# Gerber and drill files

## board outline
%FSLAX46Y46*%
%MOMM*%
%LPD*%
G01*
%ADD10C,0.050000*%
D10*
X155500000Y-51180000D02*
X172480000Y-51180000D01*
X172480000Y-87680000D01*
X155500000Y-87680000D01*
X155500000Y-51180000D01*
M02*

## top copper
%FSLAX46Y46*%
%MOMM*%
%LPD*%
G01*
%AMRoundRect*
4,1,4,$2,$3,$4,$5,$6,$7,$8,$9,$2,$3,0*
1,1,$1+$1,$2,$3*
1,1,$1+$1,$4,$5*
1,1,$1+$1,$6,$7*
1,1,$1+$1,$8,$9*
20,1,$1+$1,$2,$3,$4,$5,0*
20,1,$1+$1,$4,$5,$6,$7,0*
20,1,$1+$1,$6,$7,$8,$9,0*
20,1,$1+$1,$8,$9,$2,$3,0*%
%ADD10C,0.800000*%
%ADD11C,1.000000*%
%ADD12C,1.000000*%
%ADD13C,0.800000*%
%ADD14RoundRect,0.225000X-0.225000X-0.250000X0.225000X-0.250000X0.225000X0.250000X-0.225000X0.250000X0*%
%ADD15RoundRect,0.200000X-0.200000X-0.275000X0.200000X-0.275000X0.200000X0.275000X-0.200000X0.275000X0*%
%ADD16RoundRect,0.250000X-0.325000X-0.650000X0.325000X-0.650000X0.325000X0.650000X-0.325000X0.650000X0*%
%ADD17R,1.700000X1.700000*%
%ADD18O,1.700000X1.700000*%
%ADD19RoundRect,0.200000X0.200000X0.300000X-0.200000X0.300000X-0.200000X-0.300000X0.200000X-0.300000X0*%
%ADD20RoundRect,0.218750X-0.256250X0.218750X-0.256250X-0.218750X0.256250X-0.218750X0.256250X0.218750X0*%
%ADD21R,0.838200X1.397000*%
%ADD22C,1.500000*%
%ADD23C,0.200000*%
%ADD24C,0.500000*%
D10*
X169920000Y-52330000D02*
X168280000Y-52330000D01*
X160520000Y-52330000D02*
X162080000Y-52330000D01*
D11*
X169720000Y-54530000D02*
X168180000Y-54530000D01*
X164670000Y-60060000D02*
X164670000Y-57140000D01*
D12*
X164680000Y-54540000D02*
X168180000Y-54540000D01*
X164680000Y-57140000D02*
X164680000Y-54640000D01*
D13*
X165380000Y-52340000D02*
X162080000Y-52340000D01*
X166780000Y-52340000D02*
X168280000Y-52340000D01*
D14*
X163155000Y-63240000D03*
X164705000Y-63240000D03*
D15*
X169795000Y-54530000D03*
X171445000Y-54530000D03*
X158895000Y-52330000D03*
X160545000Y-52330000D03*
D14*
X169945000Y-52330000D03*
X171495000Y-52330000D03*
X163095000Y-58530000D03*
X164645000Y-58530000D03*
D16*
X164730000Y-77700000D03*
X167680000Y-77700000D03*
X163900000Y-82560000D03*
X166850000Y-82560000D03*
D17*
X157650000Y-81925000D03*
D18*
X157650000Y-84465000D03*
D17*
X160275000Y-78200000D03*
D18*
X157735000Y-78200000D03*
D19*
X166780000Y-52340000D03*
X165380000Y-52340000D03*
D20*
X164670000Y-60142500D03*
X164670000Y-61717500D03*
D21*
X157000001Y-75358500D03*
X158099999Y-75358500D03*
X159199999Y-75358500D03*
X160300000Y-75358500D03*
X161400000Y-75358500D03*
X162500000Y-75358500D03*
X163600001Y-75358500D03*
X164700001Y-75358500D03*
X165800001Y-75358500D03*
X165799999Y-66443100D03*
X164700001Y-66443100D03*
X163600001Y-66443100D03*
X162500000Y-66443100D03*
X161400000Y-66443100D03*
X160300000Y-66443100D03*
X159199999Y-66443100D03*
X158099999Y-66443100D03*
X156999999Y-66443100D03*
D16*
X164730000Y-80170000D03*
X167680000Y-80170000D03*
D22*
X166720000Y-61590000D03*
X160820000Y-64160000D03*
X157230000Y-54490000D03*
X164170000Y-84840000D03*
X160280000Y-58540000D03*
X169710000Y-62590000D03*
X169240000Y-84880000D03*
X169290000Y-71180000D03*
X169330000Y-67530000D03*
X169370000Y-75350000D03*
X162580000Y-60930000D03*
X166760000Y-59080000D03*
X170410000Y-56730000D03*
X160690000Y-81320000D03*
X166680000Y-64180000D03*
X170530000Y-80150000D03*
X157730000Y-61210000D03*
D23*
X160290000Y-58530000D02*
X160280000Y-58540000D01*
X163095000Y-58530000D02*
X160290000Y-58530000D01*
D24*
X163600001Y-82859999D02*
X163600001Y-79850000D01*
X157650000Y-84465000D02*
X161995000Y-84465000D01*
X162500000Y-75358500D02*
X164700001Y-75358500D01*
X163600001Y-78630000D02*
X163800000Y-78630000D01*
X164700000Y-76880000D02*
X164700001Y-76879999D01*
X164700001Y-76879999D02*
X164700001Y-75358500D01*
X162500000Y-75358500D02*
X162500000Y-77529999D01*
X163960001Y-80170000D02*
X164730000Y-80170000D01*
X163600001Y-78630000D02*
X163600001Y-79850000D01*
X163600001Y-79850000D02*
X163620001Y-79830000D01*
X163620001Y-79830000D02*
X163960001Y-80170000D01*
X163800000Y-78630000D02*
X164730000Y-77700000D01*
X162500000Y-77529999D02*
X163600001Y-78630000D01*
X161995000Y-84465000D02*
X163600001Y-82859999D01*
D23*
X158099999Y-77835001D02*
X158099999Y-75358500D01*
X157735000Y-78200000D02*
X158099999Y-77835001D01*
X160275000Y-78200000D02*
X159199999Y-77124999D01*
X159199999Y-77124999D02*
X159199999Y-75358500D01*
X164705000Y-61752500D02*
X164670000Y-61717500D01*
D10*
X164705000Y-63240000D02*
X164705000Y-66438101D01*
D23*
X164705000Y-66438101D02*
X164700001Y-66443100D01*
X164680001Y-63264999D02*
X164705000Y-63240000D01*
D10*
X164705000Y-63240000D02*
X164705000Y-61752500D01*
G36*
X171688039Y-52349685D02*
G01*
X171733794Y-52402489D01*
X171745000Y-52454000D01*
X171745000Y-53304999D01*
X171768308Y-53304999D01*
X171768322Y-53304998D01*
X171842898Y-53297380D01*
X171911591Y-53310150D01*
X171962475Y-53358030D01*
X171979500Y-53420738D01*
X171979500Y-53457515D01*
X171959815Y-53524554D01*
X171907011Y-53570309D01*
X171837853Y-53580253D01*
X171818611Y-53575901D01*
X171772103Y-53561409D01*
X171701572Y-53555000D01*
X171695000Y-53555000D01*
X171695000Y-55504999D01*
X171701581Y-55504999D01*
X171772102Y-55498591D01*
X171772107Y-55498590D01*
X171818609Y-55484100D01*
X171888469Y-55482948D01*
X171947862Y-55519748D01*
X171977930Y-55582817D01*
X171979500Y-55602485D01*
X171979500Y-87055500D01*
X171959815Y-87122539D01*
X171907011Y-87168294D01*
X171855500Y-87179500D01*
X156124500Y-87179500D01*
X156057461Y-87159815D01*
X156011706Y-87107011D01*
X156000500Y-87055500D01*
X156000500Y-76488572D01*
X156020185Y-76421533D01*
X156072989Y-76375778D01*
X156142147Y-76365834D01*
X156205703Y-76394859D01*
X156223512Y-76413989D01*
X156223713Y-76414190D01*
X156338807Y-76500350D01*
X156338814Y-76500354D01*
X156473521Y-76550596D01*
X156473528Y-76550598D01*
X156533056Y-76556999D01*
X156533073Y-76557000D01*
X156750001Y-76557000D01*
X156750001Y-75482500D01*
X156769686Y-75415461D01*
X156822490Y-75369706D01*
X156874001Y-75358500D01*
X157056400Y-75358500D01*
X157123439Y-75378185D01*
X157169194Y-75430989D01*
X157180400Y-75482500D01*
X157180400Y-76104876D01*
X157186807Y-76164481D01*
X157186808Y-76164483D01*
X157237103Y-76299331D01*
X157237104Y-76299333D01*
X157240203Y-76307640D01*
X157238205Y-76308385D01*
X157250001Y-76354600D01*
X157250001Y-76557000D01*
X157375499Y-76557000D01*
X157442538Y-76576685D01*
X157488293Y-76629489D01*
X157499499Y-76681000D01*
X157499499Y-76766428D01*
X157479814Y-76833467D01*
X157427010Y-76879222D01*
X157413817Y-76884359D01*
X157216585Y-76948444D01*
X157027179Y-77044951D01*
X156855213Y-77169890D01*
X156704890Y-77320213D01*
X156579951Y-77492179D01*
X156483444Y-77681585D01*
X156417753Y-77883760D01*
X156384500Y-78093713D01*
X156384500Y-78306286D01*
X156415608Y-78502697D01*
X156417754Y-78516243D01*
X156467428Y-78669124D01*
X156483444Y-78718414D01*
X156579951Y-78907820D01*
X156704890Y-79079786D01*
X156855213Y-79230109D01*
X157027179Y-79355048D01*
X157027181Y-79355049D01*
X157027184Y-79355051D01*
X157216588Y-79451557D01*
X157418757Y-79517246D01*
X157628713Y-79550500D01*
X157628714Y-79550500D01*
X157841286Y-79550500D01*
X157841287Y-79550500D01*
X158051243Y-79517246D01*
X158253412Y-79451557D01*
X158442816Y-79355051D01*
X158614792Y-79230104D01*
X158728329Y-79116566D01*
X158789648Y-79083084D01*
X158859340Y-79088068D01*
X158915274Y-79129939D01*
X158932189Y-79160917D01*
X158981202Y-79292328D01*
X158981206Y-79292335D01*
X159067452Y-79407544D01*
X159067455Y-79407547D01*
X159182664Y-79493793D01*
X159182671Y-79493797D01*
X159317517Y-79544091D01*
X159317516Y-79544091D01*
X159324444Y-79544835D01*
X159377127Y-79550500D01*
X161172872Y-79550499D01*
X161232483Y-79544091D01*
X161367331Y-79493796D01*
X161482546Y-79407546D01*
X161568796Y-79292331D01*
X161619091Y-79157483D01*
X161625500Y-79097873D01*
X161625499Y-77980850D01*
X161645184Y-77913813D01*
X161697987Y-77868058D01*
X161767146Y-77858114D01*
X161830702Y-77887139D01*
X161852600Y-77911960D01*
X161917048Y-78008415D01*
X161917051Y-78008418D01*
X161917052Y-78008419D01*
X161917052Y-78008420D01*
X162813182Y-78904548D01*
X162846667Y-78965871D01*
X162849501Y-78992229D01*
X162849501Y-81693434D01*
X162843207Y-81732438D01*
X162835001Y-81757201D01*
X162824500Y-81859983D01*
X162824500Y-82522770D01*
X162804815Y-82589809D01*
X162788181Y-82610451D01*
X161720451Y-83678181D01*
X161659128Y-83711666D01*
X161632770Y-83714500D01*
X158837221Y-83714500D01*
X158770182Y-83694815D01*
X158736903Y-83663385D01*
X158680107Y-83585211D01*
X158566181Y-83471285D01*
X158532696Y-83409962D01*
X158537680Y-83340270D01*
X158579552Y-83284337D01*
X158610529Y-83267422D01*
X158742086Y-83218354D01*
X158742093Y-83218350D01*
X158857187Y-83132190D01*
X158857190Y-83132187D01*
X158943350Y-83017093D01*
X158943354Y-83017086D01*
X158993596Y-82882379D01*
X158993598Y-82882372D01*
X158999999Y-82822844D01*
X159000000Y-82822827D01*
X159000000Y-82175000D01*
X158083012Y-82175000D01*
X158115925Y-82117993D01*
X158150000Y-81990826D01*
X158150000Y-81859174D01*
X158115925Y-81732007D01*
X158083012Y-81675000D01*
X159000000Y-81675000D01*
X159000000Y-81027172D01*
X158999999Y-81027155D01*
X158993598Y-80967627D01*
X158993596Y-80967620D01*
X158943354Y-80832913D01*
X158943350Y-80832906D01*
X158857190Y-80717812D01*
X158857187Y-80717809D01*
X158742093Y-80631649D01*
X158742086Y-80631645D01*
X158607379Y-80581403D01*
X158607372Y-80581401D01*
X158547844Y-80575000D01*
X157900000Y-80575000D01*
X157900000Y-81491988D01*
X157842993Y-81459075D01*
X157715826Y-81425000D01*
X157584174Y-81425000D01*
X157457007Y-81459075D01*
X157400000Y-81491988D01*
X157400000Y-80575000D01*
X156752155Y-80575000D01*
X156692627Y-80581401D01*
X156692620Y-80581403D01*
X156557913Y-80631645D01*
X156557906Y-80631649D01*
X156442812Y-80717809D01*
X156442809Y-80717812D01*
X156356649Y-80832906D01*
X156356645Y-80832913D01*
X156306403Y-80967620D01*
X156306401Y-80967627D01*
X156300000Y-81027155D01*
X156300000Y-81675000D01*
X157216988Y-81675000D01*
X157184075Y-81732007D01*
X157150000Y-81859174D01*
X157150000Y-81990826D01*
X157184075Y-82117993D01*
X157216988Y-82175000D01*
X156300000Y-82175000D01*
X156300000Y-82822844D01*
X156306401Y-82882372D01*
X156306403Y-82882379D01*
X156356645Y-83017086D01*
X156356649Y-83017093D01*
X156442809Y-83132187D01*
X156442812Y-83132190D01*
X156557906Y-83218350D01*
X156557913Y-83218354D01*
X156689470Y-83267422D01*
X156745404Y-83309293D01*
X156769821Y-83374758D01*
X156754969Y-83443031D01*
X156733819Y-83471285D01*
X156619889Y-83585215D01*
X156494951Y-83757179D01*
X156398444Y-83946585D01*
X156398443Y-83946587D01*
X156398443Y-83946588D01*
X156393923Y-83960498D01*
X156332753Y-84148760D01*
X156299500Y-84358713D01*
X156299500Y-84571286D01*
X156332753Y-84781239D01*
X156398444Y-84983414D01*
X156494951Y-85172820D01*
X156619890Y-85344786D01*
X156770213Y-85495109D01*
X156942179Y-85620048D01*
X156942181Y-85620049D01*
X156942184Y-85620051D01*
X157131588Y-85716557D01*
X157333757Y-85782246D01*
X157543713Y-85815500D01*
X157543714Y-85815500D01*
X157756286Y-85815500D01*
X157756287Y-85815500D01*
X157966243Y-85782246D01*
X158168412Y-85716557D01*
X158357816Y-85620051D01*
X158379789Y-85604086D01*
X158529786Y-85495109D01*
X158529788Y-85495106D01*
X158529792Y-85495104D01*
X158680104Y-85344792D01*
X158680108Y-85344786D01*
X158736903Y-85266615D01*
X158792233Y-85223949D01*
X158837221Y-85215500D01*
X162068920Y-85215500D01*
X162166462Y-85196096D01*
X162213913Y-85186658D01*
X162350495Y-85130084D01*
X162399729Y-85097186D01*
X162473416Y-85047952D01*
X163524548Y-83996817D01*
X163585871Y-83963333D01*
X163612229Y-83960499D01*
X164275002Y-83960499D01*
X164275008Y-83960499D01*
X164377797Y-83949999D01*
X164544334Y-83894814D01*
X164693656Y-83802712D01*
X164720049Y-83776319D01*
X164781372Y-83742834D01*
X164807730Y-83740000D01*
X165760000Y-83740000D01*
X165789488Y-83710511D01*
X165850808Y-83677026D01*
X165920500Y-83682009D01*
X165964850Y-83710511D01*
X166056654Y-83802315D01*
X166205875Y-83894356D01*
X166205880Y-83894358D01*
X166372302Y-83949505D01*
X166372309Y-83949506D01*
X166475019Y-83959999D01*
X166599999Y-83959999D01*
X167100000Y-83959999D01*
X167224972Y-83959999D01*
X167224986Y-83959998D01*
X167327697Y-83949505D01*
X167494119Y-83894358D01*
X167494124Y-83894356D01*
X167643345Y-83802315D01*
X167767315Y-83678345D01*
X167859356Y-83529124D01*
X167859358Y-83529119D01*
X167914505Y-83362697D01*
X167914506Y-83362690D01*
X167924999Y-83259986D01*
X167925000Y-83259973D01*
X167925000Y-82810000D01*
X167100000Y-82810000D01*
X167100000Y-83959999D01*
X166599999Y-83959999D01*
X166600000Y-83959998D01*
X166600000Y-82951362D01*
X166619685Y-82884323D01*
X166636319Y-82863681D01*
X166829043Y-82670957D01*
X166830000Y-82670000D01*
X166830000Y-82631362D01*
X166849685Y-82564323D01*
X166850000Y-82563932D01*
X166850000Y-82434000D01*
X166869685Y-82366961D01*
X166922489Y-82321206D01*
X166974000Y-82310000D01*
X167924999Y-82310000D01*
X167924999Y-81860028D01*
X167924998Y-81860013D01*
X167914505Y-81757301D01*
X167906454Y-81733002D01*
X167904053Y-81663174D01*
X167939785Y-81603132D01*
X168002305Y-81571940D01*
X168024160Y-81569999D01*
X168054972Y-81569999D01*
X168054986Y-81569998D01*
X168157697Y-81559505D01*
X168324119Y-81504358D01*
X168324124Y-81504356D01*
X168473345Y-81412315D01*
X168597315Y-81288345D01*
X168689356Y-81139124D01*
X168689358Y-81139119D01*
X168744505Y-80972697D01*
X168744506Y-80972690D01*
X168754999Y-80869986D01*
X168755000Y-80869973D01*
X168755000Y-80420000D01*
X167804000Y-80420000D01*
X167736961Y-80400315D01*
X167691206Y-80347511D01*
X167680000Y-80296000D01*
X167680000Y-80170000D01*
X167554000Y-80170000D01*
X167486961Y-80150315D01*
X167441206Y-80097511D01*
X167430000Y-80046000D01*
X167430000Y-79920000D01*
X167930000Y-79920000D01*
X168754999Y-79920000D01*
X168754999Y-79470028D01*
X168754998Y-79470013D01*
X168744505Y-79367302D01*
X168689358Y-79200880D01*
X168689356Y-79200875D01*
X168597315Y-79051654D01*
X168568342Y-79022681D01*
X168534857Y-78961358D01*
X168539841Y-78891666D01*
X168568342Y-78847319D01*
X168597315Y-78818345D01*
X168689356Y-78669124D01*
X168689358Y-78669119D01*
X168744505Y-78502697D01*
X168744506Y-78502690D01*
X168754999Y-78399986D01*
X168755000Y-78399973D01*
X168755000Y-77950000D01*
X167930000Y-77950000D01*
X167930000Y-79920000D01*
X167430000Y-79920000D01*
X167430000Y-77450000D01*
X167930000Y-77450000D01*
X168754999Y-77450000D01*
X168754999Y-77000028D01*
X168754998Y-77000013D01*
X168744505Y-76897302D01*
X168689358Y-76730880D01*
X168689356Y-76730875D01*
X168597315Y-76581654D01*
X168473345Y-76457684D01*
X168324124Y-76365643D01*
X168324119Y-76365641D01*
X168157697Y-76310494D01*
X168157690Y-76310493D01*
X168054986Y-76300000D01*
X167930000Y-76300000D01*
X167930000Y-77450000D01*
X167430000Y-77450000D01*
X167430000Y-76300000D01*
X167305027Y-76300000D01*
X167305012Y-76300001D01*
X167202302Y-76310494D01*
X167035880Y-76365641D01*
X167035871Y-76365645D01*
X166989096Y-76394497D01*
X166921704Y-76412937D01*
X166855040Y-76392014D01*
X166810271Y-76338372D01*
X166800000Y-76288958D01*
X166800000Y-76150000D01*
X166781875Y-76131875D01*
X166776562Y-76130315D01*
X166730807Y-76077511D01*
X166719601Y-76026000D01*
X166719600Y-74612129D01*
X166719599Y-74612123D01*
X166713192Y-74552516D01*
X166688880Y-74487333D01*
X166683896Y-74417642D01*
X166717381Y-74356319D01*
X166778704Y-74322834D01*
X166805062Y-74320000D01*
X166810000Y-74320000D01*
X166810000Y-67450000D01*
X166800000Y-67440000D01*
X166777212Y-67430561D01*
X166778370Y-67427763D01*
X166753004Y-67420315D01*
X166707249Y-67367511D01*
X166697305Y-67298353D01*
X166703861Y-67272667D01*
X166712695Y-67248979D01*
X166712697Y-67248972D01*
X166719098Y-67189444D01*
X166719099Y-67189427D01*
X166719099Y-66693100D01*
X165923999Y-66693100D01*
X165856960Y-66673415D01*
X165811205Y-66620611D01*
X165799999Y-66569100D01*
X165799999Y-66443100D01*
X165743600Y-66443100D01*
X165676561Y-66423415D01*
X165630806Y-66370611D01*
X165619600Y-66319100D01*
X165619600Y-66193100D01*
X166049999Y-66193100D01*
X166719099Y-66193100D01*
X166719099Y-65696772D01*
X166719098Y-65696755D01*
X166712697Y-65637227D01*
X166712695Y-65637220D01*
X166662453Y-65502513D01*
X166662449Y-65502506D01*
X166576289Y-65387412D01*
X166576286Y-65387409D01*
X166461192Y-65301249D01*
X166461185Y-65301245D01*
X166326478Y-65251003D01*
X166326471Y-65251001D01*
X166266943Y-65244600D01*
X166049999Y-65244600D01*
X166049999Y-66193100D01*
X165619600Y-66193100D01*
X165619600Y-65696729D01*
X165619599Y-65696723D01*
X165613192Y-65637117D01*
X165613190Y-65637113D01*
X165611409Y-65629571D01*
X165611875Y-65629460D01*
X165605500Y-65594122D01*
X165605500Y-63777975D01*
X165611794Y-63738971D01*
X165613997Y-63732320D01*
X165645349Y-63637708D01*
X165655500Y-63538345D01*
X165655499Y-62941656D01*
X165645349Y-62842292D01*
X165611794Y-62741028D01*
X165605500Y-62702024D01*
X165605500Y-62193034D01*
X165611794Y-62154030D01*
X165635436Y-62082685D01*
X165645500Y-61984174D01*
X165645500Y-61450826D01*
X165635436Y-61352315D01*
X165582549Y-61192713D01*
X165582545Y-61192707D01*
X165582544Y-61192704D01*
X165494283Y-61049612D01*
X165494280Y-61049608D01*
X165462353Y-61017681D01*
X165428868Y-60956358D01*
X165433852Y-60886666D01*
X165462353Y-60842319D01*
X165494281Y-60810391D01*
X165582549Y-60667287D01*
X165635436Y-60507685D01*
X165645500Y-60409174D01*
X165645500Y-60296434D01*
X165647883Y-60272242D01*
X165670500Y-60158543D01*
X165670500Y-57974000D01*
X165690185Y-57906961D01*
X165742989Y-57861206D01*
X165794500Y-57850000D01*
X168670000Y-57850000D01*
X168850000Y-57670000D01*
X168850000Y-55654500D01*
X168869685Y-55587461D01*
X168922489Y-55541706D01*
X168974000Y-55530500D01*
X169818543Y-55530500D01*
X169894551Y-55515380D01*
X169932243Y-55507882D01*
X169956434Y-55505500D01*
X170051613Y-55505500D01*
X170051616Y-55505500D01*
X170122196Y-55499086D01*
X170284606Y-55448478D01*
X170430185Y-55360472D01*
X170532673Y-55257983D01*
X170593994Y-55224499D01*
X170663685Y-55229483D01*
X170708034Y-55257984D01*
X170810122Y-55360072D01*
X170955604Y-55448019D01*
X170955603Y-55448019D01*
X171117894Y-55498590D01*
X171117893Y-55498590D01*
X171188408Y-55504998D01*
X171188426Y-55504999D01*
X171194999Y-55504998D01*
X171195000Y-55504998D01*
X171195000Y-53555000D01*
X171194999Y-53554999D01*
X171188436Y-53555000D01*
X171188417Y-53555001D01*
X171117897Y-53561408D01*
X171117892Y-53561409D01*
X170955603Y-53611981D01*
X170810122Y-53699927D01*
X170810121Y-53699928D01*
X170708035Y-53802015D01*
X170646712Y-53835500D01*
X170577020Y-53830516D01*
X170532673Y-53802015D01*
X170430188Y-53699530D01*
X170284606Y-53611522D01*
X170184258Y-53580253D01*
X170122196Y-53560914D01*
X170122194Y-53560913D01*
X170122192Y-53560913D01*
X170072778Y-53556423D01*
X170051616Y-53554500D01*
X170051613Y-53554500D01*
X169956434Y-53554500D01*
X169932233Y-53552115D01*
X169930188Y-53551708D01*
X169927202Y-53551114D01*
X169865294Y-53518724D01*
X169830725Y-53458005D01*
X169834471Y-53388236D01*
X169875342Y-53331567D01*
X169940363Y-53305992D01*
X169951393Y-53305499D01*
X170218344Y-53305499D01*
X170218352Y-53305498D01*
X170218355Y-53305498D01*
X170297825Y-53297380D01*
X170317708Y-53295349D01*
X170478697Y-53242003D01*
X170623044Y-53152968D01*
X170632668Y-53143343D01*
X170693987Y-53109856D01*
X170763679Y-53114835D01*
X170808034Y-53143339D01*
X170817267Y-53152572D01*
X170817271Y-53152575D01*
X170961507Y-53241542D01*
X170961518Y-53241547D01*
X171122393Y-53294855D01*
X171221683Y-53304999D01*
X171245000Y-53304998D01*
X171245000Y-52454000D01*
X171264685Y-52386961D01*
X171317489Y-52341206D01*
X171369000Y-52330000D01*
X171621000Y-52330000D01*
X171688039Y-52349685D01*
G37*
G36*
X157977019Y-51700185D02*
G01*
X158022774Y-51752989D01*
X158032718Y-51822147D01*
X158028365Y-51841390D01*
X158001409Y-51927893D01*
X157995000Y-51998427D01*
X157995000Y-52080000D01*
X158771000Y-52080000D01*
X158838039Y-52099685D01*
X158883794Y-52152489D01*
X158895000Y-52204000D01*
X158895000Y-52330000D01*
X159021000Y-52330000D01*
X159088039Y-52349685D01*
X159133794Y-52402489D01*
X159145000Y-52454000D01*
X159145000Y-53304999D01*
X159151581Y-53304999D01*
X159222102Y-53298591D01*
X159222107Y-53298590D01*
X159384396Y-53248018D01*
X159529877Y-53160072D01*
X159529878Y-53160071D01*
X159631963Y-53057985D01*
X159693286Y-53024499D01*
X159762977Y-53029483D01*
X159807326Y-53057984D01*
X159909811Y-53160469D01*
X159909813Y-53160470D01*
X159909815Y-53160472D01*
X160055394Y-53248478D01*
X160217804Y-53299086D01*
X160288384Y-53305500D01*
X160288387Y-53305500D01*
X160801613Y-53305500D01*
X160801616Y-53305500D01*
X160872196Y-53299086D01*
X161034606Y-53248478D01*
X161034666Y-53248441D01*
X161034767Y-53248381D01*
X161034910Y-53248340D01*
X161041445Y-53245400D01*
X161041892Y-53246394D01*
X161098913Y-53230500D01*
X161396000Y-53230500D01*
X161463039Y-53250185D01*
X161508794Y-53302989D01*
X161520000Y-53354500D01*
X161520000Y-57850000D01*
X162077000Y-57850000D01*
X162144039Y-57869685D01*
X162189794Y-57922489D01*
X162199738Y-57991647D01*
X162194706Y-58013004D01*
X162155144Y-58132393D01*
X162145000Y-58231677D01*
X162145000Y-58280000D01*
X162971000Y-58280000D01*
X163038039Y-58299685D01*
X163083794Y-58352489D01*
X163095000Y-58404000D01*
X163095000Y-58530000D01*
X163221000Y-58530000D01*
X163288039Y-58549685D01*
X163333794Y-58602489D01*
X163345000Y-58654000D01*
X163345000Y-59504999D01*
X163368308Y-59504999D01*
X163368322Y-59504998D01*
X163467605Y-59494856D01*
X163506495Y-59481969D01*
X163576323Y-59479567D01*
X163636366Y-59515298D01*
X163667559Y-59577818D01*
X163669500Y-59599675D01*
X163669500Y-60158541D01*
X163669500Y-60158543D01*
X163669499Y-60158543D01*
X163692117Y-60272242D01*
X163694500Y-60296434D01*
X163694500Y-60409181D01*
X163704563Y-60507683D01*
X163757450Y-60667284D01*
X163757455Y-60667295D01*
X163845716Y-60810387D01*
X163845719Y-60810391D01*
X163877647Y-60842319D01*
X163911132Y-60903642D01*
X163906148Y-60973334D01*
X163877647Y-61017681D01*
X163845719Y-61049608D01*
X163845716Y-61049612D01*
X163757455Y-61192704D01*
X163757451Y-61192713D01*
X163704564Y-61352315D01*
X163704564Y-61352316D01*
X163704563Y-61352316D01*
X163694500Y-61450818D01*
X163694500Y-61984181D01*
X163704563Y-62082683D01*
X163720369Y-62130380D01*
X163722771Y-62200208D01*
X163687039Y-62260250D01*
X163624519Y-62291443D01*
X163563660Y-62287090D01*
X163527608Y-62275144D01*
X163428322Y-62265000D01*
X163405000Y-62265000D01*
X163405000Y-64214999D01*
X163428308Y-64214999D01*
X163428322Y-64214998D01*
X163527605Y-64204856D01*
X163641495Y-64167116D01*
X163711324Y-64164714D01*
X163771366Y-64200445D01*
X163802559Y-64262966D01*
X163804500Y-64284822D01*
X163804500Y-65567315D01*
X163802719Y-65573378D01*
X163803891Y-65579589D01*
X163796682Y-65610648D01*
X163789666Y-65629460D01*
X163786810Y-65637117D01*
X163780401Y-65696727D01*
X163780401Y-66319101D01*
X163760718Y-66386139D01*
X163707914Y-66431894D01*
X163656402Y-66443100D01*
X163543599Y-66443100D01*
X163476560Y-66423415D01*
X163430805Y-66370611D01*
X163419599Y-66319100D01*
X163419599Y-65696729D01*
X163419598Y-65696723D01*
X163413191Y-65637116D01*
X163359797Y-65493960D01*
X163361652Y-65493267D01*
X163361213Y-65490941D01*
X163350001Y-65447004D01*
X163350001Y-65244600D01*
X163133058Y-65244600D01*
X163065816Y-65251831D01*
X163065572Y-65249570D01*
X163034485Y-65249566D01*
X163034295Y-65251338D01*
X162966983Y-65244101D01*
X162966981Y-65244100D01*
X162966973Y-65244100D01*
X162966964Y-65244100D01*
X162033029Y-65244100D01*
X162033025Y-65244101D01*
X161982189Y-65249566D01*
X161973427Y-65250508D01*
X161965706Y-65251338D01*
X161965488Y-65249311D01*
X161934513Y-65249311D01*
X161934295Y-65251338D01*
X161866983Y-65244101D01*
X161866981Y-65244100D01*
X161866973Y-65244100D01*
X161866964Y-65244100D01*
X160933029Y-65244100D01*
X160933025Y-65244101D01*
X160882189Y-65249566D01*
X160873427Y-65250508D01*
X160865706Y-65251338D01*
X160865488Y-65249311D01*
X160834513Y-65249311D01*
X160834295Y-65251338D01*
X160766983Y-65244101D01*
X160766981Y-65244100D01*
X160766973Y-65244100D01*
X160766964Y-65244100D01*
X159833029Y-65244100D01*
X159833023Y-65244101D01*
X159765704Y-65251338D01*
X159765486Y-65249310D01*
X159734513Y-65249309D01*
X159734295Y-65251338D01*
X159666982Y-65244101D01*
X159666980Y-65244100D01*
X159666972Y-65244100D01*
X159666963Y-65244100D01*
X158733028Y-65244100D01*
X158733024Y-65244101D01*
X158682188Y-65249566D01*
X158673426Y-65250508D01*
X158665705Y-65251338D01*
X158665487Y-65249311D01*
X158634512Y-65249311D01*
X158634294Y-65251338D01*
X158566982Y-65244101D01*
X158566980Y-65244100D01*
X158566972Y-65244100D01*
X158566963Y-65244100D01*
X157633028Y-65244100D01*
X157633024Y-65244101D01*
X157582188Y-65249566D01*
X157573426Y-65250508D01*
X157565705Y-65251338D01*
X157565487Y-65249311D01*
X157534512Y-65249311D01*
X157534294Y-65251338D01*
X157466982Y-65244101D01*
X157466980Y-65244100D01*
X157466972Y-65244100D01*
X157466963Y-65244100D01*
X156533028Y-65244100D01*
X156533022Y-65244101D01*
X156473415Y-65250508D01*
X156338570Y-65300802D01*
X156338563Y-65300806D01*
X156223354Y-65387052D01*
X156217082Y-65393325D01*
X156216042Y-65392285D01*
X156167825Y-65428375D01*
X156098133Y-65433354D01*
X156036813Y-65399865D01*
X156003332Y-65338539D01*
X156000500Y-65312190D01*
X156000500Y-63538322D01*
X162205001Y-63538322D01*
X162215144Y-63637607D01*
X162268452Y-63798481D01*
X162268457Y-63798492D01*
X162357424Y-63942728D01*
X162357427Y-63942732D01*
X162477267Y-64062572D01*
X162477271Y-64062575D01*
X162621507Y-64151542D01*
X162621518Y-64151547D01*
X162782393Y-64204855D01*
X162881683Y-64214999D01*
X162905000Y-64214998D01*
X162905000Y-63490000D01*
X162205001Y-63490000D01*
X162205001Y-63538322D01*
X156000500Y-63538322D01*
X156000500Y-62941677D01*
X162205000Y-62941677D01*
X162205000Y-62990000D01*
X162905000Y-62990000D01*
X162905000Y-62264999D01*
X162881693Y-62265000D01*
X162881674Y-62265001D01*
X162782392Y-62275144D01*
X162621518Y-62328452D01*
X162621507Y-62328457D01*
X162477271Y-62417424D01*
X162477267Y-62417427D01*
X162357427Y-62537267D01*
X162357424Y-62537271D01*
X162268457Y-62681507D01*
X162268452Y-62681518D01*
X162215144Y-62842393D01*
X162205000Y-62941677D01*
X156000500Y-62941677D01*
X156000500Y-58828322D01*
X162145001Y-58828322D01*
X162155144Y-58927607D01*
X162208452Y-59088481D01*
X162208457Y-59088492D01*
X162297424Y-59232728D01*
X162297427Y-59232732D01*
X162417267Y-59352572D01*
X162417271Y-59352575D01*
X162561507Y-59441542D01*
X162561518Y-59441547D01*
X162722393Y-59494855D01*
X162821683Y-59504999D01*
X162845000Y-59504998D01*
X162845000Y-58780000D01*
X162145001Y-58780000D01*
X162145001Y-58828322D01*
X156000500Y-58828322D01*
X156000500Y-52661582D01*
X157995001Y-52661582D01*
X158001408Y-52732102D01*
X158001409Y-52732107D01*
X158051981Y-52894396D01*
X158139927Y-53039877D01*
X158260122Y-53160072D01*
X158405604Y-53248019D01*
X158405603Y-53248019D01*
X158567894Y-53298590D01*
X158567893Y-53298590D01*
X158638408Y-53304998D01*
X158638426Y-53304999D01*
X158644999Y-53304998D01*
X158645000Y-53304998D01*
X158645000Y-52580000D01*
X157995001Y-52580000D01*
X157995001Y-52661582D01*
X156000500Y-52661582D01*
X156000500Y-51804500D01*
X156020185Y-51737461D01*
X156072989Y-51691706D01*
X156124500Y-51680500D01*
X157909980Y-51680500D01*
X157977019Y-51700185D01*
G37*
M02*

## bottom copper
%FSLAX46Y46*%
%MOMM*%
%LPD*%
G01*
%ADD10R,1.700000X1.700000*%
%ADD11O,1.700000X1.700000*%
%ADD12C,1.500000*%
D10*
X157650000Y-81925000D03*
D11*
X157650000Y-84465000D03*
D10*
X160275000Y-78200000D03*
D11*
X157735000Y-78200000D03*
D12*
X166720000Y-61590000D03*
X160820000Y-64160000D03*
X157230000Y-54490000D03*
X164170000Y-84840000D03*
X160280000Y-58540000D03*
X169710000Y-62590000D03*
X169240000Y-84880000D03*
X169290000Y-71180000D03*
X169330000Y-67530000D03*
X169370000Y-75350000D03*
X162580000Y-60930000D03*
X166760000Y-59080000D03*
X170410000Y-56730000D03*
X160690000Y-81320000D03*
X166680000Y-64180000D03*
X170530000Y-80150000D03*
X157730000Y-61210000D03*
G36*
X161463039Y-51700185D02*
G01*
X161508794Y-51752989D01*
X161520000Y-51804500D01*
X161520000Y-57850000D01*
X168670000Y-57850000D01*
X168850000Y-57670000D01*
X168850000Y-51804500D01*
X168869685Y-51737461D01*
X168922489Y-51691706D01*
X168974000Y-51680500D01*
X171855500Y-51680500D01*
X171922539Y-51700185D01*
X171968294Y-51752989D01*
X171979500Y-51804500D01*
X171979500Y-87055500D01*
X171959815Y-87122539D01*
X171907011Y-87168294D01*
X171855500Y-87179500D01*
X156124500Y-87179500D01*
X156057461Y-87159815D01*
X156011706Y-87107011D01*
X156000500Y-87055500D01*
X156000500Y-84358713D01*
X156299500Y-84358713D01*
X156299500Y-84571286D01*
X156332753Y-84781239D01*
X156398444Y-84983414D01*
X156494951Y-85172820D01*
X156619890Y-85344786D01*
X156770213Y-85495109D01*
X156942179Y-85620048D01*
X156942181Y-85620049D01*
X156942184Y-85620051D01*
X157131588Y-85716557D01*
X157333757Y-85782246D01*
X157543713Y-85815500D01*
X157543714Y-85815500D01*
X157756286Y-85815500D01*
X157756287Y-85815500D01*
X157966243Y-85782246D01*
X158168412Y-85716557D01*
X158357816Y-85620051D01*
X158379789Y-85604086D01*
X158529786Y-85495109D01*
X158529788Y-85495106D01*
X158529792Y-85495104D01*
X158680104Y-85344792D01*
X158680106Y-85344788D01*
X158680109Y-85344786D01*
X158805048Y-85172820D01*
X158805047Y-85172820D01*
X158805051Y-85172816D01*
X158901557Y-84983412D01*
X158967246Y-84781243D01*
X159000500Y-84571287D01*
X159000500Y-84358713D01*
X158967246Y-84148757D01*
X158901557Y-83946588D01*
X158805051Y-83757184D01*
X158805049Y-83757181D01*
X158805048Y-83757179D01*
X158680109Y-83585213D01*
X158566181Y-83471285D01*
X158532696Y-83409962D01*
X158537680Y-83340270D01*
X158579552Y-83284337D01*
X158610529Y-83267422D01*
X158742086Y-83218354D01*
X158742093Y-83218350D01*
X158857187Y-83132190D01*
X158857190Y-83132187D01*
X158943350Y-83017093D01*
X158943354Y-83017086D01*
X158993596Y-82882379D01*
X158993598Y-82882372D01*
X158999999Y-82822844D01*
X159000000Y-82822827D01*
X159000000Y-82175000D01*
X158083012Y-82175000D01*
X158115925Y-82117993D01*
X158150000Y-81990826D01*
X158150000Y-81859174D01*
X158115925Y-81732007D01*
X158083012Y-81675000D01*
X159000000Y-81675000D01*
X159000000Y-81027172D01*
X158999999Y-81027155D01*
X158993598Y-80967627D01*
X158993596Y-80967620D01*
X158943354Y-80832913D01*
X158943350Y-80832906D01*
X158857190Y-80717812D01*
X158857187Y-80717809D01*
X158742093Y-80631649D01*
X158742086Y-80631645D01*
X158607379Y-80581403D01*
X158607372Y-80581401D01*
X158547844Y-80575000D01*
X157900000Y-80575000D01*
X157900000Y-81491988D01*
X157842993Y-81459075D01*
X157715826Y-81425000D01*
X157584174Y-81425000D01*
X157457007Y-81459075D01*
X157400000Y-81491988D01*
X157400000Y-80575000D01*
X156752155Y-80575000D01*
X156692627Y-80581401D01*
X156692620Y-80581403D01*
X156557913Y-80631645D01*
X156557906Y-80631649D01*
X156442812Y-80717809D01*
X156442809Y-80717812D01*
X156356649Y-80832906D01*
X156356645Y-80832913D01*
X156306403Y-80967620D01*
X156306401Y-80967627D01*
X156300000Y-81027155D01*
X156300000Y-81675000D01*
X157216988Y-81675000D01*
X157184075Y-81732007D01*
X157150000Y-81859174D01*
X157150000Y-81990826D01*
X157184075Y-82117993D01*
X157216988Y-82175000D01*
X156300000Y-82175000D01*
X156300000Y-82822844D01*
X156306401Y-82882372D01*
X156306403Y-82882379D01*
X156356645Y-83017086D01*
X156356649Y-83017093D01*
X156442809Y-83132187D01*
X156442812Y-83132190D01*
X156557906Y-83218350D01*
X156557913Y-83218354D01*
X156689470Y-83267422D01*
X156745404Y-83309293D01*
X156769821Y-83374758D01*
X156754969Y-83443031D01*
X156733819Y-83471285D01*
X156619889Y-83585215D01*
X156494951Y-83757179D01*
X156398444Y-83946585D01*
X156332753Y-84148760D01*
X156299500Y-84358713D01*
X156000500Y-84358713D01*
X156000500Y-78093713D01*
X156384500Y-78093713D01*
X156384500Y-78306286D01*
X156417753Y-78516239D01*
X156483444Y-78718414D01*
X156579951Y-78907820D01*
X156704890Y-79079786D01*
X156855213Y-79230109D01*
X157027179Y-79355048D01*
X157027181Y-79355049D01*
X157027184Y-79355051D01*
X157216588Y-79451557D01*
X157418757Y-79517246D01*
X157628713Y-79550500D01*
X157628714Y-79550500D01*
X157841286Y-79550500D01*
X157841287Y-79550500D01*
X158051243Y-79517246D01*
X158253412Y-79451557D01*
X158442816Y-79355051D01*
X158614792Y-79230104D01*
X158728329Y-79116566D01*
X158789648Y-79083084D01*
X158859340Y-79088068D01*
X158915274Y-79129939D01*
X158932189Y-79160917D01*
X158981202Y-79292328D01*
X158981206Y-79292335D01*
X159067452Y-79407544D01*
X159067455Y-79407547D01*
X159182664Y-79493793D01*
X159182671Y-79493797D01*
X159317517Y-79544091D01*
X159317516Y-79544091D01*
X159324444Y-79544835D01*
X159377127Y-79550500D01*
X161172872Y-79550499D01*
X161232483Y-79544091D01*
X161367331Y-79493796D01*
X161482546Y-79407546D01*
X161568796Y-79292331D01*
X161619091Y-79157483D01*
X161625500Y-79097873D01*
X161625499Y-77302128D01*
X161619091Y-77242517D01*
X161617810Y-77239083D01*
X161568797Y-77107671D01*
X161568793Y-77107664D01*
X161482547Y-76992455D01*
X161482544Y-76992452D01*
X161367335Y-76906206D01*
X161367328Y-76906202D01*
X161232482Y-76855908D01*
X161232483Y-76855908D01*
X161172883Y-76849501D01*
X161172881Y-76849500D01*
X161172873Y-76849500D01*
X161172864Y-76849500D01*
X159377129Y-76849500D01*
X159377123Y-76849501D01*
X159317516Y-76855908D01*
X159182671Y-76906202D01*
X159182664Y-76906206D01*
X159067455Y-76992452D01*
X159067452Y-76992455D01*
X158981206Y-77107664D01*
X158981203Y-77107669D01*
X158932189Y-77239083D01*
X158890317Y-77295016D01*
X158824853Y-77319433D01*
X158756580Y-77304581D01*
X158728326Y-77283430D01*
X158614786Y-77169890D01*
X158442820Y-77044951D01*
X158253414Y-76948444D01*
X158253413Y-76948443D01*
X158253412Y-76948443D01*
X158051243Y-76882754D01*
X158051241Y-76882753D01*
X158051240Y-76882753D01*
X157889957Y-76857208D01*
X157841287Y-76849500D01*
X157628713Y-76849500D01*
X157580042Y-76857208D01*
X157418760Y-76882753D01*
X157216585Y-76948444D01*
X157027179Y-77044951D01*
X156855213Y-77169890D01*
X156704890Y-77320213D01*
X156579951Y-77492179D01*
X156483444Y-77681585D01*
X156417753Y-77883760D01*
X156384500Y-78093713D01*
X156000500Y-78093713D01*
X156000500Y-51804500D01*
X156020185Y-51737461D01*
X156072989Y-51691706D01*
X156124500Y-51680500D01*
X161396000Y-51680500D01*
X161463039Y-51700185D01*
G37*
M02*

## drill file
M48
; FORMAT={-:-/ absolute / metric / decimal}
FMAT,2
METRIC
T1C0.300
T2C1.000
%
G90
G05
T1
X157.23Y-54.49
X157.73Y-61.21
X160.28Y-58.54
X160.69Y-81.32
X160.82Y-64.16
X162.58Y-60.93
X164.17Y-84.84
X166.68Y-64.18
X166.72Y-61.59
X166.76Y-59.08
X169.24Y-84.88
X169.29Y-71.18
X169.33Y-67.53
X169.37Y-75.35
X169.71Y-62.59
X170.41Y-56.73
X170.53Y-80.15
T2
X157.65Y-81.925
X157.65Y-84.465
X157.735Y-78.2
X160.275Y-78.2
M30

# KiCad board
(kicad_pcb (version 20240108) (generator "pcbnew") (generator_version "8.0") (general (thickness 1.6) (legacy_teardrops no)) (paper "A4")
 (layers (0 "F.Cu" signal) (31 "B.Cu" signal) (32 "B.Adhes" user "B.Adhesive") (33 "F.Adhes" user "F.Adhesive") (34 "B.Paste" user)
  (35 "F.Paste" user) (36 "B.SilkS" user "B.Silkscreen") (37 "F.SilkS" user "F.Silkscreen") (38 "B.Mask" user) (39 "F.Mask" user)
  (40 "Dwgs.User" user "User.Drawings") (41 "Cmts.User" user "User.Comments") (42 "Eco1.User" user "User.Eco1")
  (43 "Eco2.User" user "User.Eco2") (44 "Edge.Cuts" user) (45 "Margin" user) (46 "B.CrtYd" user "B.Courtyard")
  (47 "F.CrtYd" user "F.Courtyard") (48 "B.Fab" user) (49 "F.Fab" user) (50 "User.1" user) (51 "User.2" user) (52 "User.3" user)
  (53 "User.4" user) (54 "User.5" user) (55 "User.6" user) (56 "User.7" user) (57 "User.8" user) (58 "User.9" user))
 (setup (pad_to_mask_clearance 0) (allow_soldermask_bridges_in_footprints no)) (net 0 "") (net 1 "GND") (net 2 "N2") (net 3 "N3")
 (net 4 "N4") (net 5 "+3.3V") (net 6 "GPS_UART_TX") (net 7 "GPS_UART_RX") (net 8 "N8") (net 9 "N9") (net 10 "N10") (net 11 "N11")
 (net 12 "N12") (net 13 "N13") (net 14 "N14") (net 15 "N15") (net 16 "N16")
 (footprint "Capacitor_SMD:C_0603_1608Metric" (layer "F.Cu") (at 163.93 63.24)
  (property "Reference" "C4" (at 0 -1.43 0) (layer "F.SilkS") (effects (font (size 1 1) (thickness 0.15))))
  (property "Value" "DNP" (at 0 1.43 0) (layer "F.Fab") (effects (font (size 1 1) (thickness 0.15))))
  (pad "1" smd roundrect (at -0.775 0) (size 0.9 0.95) (layers "F.Cu" "F.Paste" "F.Mask") (roundrect_rratio 0.25) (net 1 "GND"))
  (pad "2" smd roundrect (at 0.775 0) (size 0.9 0.95) (layers "F.Cu" "F.Paste" "F.Mask") (roundrect_rratio 0.25) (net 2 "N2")))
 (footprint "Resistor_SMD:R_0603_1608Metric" (layer "F.Cu") (at 170.62 54.53)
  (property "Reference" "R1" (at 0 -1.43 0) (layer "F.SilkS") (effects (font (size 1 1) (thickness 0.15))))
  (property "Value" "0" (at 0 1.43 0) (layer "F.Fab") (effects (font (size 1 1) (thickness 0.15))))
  (pad "1" smd roundrect (at -0.825 0) (size 0.8 0.95) (layers "F.Cu" "F.Paste" "F.Mask") (roundrect_rratio 0.25) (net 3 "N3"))
  (pad "2" smd roundrect (at 0.825 0) (size 0.8 0.95) (layers "F.Cu" "F.Paste" "F.Mask") (roundrect_rratio 0.25) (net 1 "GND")))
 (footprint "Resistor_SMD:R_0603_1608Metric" (layer "F.Cu") (at 159.72 52.33)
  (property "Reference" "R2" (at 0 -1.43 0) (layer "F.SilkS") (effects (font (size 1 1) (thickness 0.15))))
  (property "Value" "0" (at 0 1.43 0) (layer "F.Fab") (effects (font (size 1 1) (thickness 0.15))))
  (pad "1" smd roundrect (at -0.825 0) (size 0.8 0.95) (layers "F.Cu" "F.Paste" "F.Mask") (roundrect_rratio 0.25) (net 1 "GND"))
  (pad "2" smd roundrect (at 0.825 0) (size 0.8 0.95) (layers "F.Cu" "F.Paste" "F.Mask") (roundrect_rratio 0.25) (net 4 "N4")))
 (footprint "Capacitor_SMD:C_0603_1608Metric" (layer "F.Cu") (at 170.72 52.33)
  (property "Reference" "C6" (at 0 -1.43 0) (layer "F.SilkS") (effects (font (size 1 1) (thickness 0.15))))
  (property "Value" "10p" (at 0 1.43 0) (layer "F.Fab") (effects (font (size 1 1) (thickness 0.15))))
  (pad "1" smd roundrect (at -0.775 0) (size 0.9 0.95) (layers "F.Cu" "F.Paste" "F.Mask") (roundrect_rratio 0.25) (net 4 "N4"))
  (pad "2" smd roundrect (at 0.775 0) (size 0.9 0.95) (layers "F.Cu" "F.Paste" "F.Mask") (roundrect_rratio 0.25) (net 1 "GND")))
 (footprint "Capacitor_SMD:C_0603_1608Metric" (layer "F.Cu") (at 163.87 58.53)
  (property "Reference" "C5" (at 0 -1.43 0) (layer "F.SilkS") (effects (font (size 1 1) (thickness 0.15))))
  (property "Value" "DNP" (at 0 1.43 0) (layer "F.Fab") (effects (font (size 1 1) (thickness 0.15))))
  (pad "1" smd roundrect (at -0.775 0) (size 0.9 0.95) (layers "F.Cu" "F.Paste" "F.Mask") (roundrect_rratio 0.25) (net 1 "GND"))
  (pad "2" smd roundrect (at 0.775 0) (size 0.9 0.95) (layers "F.Cu" "F.Paste" "F.Mask") (roundrect_rratio 0.25) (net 3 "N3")))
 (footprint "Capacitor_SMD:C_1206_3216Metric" (layer "F.Cu") (at 166.205 77.7)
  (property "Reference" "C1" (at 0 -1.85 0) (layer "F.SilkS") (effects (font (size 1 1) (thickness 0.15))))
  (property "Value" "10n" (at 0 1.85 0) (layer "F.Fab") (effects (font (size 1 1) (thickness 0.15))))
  (pad "1" smd roundrect (at -1.475 0) (size 1.15 1.8) (layers "F.Cu" "F.Paste" "F.Mask") (roundrect_rratio 0.217391) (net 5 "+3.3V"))
  (pad "2" smd roundrect (at 1.475 0) (size 1.15 1.8) (layers "F.Cu" "F.Paste" "F.Mask") (roundrect_rratio 0.217391) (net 1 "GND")))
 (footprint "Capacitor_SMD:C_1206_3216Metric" (layer "F.Cu") (at 165.375 82.56)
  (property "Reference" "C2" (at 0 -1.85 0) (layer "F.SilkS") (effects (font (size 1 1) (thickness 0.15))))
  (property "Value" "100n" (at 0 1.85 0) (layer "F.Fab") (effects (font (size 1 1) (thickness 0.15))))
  (pad "1" smd roundrect (at -1.475 0) (size 1.15 1.8) (layers "F.Cu" "F.Paste" "F.Mask") (roundrect_rratio 0.217391) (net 5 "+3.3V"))
  (pad "2" smd roundrect (at 1.475 0) (size 1.15 1.8) (layers "F.Cu" "F.Paste" "F.Mask") (roundrect_rratio 0.217391) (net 1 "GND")))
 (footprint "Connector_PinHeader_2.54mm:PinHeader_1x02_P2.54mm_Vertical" (layer "F.Cu") (at 157.65 81.925)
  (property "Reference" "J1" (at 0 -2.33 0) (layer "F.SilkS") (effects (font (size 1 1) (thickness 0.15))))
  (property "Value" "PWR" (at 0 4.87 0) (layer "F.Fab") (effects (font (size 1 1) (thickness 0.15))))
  (pad "1" thru_hole rect (at 0 0) (size 1.7 1.7) (drill 1) (layers "*.Cu" "*.Mask") (remove_unused_layers no) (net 1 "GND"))
  (pad "2" thru_hole oval (at 0 2.54) (size 1.7 1.7) (drill 1) (layers "*.Cu" "*.Mask") (remove_unused_layers no) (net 5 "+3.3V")))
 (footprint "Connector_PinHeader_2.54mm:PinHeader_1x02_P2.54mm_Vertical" (layer "F.Cu") (at 160.275 78.2 -90)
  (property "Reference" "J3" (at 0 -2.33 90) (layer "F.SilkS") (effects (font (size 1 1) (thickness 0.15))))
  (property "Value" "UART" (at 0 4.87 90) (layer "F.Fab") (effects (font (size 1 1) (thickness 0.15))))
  (pad "1" thru_hole rect (at 0 0 270) (size 1.7 1.7) (drill 1) (layers "*.Cu" "*.Mask") (remove_unused_layers no) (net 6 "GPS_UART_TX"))
  (pad "2" thru_hole oval (at 0 2.54 270) (size 1.7 1.7) (drill 1) (layers "*.Cu" "*.Mask") (remove_unused_layers no) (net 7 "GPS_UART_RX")))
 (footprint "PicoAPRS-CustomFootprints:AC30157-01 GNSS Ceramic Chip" (layer "F.Cu") (at 165.18 54.64)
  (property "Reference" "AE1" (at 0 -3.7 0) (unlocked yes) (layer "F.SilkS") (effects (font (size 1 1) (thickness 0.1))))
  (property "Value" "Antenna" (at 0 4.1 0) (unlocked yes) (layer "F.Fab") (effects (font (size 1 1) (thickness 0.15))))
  (fp_line (start -0.5 -0.1) (end 3 -0.1) (stroke (width 1) (type default)) (layer "F.Cu"))
  (fp_line (start -0.5 2.5) (end -0.5 0) (stroke (width 1) (type default)) (layer "F.Cu"))
  (fp_line (start 0.2 -2.3) (end -3.1 -2.3) (stroke (width 0.8) (type default)) (layer "F.Cu"))
  (fp_line (start 1.6 -2.3) (end 3.1 -2.3) (stroke (width 0.8) (type default)) (layer "F.Cu"))
  (pad "1" smd roundrect (at 1.6 -2.3 180) (size 0.8 1) (layers "F.Cu" "F.Paste" "F.Mask") (roundrect_rratio 0.25) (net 4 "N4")
   (thermal_bridge_angle 45))
  (pad "2" smd roundrect (at 0.2 -2.3 180) (size 0.8 1) (layers "F.Cu" "F.Paste" "F.Mask") (roundrect_rratio 0.25) (thermal_bridge_angle 45)))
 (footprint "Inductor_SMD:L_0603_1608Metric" (layer "F.Cu") (at 164.67 60.93 -90)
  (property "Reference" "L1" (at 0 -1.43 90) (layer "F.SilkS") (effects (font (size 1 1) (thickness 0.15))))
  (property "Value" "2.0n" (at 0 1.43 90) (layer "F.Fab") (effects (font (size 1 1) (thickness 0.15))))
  (pad "1" smd roundrect (at -0.7875 0 270) (size 0.875 0.95) (layers "F.Cu" "F.Paste" "F.Mask") (roundrect_rratio 0.25) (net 3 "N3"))
  (pad "2" smd roundrect (at 0.7875 0 270) (size 0.875 0.95) (layers "F.Cu" "F.Paste" "F.Mask") (roundrect_rratio 0.25) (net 2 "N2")))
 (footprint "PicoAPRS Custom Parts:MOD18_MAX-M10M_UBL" (layer "F.Cu") (at 161.4 70.9008 90)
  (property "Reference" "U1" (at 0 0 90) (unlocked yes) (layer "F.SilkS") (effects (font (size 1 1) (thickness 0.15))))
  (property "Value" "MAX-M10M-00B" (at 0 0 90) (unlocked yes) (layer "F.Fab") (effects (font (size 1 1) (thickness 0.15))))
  (pad "1" smd rect (at -4.4577 -4.399999 90) (size 1.397 0.8382) (layers "F.Cu" "F.Paste" "F.Mask") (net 1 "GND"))
  (pad "2" smd rect (at -4.4577 -3.300001 90) (size 1.397 0.8382) (layers "F.Cu" "F.Paste" "F.Mask") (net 7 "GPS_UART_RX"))
  (pad "3" smd rect (at -4.4577 -2.200001 90) (size 1.397 0.8382) (layers "F.Cu" "F.Paste" "F.Mask") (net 6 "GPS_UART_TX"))
  (pad "4" smd rect (at -4.4577 -1.1 90) (size 1.397 0.8382) (layers "F.Cu" "F.Paste" "F.Mask") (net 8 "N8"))
  (pad "5" smd rect (at -4.4577 0 90) (size 1.397 0.8382) (layers "F.Cu" "F.Paste" "F.Mask") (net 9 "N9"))
  (pad "6" smd rect (at -4.4577 1.1 90) (size 1.397 0.8382) (layers "F.Cu" "F.Paste" "F.Mask") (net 5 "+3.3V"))
  (pad "7" smd rect (at -4.4577 2.200001 90) (size 1.397 0.8382) (layers "F.Cu" "F.Paste" "F.Mask") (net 5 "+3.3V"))
  (pad "8" smd rect (at -4.4577 3.300001 90) (size 1.397 0.8382) (layers "F.Cu" "F.Paste" "F.Mask") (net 5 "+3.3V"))
  (pad "9" smd rect (at -4.4577 4.400001 90) (size 1.397 0.8382) (layers "F.Cu" "F.Paste" "F.Mask") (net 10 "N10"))
  (pad "10" smd rect (at 4.4577 4.399999 90) (size 1.397 0.8382) (layers "F.Cu" "F.Paste" "F.Mask") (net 1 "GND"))
  (pad "11" smd rect (at 4.4577 3.300001 90) (size 1.397 0.8382) (layers "F.Cu" "F.Paste" "F.Mask") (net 2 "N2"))
  (pad "12" smd rect (at 4.4577 2.200001 90) (size 1.397 0.8382) (layers "F.Cu" "F.Paste" "F.Mask") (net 1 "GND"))
  (pad "13" smd rect (at 4.4577 1.1 90) (size 1.397 0.8382) (layers "F.Cu" "F.Paste" "F.Mask") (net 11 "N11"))
  (pad "14" smd rect (at 4.4577 0 90) (size 1.397 0.8382) (layers "F.Cu" "F.Paste" "F.Mask") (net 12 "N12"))
  (pad "15" smd rect (at 4.4577 -1.1 90) (size 1.397 0.8382) (layers "F.Cu" "F.Paste" "F.Mask") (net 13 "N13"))
  (pad "16" smd rect (at 4.4577 -2.200001 90) (size 1.397 0.8382) (layers "F.Cu" "F.Paste" "F.Mask") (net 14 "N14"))
  (pad "17" smd rect (at 4.4577 -3.300001 90) (size 1.397 0.8382) (layers "F.Cu" "F.Paste" "F.Mask") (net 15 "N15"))
  (pad "18" smd rect (at 4.4577 -4.400001 90) (size 1.397 0.8382) (layers "F.Cu" "F.Paste" "F.Mask") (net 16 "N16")))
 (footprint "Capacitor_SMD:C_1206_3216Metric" (layer "F.Cu") (at 166.205 80.17)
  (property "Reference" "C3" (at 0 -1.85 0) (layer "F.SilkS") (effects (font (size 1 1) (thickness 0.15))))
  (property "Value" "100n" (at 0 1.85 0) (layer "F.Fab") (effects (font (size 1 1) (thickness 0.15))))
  (pad "1" smd roundrect (at -1.475 0) (size 1.15 1.8) (layers "F.Cu" "F.Paste" "F.Mask") (roundrect_rratio 0.217391) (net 5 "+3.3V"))
  (pad "2" smd roundrect (at 1.475 0) (size 1.15 1.8) (layers "F.Cu" "F.Paste" "F.Mask") (roundrect_rratio 0.217391) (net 1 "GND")))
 (gr_line (start 169.92 52.33) (end 168.28 52.33) (stroke (width 0.8) (type default)) (layer "F.Cu") (net 4))
 (gr_line (start 160.52 52.33) (end 162.08 52.33) (stroke (width 0.8) (type default)) (layer "F.Cu") (net 4))
 (gr_line (start 169.72 54.53) (end 168.18 54.53) (stroke (width 1) (type default)) (layer "F.Cu") (net 3))
 (gr_line (start 164.67 60.06) (end 164.67 57.14) (stroke (width 1) (type default)) (layer "F.Cu") (net 3))
 (gr_rect (start 155.5 51.18) (end 172.48 87.68) (stroke (width 0.05) (type default)) (fill none) (layer "Edge.Cuts"))
 (segment (start 160.29 58.53) (end 160.28 58.54) (width 0.2) (layer "F.Cu") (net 1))
 (segment (start 163.095 58.53) (end 160.29 58.53) (width 0.2) (layer "F.Cu") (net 1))
 (via (at 166.72 61.59) (size 1.5) (drill 0.3) (layers "F.Cu" "B.Cu") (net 1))
 (via (at 160.82 64.16) (size 1.5) (drill 0.3) (layers "F.Cu" "B.Cu") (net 1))
 (via (at 157.23 54.49) (size 1.5) (drill 0.3) (layers "F.Cu" "B.Cu") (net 1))
 (via (at 164.17 84.84) (size 1.5) (drill 0.3) (layers "F.Cu" "B.Cu") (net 1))
 (via (at 160.28 58.54) (size 1.5) (drill 0.3) (layers "F.Cu" "B.Cu") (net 1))
 (via (at 169.71 62.59) (size 1.5) (drill 0.3) (layers "F.Cu" "B.Cu") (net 1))
 (via (at 169.24 84.88) (size 1.5) (drill 0.3) (layers "F.Cu" "B.Cu") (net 1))
 (via (at 169.29 71.18) (size 1.5) (drill 0.3) (layers "F.Cu" "B.Cu") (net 1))
 (via (at 169.33 67.53) (size 1.5) (drill 0.3) (layers "F.Cu" "B.Cu") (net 1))
 (via (at 169.37 75.35) (size 1.5) (drill 0.3) (layers "F.Cu" "B.Cu") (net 1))
 (via (at 162.58 60.93) (size 1.5) (drill 0.3) (layers "F.Cu" "B.Cu") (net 1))
 (via (at 166.76 59.08) (size 1.5) (drill 0.3) (layers "F.Cu" "B.Cu") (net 1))
 (via (at 170.41 56.73) (size 1.5) (drill 0.3) (layers "F.Cu" "B.Cu") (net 1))
 (via (at 160.69 81.32) (size 1.5) (drill 0.3) (layers "F.Cu" "B.Cu") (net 1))
 (via (at 166.68 64.18) (size 1.5) (drill 0.3) (layers "F.Cu" "B.Cu") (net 1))
 (via (at 170.53 80.15) (size 1.5) (drill 0.3) (layers "F.Cu" "B.Cu") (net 1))
 (via (at 157.73 61.21) (size 1.5) (drill 0.3) (layers "F.Cu" "B.Cu") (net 1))
 (segment (start 163.600001 82.859999) (end 163.600001 79.85) (width 0.5) (layer "F.Cu") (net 5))
 (segment (start 157.65 84.465) (end 161.995 84.465) (width 0.5) (layer "F.Cu") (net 5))
 (segment (start 162.5 75.3585) (end 164.700001 75.3585) (width 0.5) (layer "F.Cu") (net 5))
 (segment (start 163.600001 78.63) (end 163.8 78.63) (width 0.5) (layer "F.Cu") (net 5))
 (segment (start 164.7 76.88) (end 164.700001 76.879999) (width 0.5) (layer "F.Cu") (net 5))
 (segment (start 164.700001 76.879999) (end 164.700001 75.3585) (width 0.5) (layer "F.Cu") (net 5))
 (segment (start 162.5 75.3585) (end 162.5 77.529999) (width 0.5) (layer "F.Cu") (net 5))
 (segment (start 163.960001 80.17) (end 164.73 80.17) (width 0.5) (layer "F.Cu") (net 5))
 (segment (start 163.600001 78.63) (end 163.600001 79.85) (width 0.5) (layer "F.Cu") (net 5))
 (segment (start 163.600001 79.85) (end 163.620001 79.83) (width 0.5) (layer "F.Cu") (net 5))
 (segment (start 163.620001 79.83) (end 163.960001 80.17) (width 0.5) (layer "F.Cu") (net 5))
 (segment (start 163.8 78.63) (end 164.73 77.7) (width 0.5) (layer "F.Cu") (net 5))
 (segment (start 162.5 77.529999) (end 163.600001 78.63) (width 0.5) (layer "F.Cu") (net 5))
 (segment (start 161.995 84.465) (end 163.600001 82.859999) (width 0.5) (layer "F.Cu") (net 5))
 (segment (start 158.099999 77.835001) (end 158.099999 75.3585) (width 0.2) (layer "F.Cu") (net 7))
 (segment (start 157.735 78.2) (end 158.099999 77.835001) (width 0.2) (layer "F.Cu") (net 7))
 (segment (start 160.275 78.2) (end 159.199999 77.124999) (width 0.2) (layer "F.Cu") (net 6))
 (segment (start 159.199999 77.124999) (end 159.199999 75.3585) (width 0.2) (layer "F.Cu") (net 6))
 (segment (start 164.705 61.7525) (end 164.67 61.7175) (width 0.2) (layer "F.Cu") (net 2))
 (segment (start 164.705 63.24) (end 164.705 66.438101) (width 0.8) (layer "F.Cu") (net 2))
 (segment (start 164.705 66.438101) (end 164.700001 66.4431) (width 0.2) (layer "F.Cu") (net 2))
 (segment (start 164.680001 63.264999) (end 164.705 63.24) (width 0.2) (layer "F.Cu") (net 2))
 (segment (start 164.705 63.24) (end 164.705 61.7525) (width 0.8) (layer "F.Cu") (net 2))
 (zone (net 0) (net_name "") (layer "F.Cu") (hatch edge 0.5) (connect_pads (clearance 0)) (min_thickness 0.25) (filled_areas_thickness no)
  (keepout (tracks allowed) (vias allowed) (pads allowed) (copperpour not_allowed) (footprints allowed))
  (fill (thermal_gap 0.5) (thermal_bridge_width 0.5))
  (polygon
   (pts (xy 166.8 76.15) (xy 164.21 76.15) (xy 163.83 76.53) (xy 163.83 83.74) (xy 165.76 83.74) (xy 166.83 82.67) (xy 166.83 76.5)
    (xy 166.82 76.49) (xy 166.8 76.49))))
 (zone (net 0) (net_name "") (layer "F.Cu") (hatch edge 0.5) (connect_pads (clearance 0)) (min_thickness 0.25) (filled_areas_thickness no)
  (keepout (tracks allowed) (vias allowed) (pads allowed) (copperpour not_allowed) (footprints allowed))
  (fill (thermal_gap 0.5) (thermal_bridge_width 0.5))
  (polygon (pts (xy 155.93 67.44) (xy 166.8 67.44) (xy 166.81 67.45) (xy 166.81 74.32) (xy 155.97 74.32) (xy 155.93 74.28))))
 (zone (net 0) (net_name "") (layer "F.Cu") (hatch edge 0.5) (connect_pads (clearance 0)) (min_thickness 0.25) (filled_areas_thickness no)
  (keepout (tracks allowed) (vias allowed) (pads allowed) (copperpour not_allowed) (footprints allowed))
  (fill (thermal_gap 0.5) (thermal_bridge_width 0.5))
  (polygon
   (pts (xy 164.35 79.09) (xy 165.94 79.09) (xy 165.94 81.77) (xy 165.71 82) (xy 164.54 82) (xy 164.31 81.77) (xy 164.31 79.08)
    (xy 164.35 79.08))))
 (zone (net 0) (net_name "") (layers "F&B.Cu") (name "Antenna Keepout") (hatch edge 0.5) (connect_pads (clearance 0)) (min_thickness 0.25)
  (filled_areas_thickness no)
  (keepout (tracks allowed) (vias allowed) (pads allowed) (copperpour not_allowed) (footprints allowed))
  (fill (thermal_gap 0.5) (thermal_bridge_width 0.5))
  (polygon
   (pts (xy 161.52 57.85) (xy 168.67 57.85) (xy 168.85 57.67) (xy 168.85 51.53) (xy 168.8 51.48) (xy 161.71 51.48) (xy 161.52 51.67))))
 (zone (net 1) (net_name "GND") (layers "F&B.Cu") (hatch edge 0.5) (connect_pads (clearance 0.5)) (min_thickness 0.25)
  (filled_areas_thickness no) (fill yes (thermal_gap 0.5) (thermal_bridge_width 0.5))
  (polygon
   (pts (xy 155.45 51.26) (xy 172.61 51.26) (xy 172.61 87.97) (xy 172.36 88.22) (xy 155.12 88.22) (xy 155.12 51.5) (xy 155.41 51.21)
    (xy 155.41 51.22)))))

